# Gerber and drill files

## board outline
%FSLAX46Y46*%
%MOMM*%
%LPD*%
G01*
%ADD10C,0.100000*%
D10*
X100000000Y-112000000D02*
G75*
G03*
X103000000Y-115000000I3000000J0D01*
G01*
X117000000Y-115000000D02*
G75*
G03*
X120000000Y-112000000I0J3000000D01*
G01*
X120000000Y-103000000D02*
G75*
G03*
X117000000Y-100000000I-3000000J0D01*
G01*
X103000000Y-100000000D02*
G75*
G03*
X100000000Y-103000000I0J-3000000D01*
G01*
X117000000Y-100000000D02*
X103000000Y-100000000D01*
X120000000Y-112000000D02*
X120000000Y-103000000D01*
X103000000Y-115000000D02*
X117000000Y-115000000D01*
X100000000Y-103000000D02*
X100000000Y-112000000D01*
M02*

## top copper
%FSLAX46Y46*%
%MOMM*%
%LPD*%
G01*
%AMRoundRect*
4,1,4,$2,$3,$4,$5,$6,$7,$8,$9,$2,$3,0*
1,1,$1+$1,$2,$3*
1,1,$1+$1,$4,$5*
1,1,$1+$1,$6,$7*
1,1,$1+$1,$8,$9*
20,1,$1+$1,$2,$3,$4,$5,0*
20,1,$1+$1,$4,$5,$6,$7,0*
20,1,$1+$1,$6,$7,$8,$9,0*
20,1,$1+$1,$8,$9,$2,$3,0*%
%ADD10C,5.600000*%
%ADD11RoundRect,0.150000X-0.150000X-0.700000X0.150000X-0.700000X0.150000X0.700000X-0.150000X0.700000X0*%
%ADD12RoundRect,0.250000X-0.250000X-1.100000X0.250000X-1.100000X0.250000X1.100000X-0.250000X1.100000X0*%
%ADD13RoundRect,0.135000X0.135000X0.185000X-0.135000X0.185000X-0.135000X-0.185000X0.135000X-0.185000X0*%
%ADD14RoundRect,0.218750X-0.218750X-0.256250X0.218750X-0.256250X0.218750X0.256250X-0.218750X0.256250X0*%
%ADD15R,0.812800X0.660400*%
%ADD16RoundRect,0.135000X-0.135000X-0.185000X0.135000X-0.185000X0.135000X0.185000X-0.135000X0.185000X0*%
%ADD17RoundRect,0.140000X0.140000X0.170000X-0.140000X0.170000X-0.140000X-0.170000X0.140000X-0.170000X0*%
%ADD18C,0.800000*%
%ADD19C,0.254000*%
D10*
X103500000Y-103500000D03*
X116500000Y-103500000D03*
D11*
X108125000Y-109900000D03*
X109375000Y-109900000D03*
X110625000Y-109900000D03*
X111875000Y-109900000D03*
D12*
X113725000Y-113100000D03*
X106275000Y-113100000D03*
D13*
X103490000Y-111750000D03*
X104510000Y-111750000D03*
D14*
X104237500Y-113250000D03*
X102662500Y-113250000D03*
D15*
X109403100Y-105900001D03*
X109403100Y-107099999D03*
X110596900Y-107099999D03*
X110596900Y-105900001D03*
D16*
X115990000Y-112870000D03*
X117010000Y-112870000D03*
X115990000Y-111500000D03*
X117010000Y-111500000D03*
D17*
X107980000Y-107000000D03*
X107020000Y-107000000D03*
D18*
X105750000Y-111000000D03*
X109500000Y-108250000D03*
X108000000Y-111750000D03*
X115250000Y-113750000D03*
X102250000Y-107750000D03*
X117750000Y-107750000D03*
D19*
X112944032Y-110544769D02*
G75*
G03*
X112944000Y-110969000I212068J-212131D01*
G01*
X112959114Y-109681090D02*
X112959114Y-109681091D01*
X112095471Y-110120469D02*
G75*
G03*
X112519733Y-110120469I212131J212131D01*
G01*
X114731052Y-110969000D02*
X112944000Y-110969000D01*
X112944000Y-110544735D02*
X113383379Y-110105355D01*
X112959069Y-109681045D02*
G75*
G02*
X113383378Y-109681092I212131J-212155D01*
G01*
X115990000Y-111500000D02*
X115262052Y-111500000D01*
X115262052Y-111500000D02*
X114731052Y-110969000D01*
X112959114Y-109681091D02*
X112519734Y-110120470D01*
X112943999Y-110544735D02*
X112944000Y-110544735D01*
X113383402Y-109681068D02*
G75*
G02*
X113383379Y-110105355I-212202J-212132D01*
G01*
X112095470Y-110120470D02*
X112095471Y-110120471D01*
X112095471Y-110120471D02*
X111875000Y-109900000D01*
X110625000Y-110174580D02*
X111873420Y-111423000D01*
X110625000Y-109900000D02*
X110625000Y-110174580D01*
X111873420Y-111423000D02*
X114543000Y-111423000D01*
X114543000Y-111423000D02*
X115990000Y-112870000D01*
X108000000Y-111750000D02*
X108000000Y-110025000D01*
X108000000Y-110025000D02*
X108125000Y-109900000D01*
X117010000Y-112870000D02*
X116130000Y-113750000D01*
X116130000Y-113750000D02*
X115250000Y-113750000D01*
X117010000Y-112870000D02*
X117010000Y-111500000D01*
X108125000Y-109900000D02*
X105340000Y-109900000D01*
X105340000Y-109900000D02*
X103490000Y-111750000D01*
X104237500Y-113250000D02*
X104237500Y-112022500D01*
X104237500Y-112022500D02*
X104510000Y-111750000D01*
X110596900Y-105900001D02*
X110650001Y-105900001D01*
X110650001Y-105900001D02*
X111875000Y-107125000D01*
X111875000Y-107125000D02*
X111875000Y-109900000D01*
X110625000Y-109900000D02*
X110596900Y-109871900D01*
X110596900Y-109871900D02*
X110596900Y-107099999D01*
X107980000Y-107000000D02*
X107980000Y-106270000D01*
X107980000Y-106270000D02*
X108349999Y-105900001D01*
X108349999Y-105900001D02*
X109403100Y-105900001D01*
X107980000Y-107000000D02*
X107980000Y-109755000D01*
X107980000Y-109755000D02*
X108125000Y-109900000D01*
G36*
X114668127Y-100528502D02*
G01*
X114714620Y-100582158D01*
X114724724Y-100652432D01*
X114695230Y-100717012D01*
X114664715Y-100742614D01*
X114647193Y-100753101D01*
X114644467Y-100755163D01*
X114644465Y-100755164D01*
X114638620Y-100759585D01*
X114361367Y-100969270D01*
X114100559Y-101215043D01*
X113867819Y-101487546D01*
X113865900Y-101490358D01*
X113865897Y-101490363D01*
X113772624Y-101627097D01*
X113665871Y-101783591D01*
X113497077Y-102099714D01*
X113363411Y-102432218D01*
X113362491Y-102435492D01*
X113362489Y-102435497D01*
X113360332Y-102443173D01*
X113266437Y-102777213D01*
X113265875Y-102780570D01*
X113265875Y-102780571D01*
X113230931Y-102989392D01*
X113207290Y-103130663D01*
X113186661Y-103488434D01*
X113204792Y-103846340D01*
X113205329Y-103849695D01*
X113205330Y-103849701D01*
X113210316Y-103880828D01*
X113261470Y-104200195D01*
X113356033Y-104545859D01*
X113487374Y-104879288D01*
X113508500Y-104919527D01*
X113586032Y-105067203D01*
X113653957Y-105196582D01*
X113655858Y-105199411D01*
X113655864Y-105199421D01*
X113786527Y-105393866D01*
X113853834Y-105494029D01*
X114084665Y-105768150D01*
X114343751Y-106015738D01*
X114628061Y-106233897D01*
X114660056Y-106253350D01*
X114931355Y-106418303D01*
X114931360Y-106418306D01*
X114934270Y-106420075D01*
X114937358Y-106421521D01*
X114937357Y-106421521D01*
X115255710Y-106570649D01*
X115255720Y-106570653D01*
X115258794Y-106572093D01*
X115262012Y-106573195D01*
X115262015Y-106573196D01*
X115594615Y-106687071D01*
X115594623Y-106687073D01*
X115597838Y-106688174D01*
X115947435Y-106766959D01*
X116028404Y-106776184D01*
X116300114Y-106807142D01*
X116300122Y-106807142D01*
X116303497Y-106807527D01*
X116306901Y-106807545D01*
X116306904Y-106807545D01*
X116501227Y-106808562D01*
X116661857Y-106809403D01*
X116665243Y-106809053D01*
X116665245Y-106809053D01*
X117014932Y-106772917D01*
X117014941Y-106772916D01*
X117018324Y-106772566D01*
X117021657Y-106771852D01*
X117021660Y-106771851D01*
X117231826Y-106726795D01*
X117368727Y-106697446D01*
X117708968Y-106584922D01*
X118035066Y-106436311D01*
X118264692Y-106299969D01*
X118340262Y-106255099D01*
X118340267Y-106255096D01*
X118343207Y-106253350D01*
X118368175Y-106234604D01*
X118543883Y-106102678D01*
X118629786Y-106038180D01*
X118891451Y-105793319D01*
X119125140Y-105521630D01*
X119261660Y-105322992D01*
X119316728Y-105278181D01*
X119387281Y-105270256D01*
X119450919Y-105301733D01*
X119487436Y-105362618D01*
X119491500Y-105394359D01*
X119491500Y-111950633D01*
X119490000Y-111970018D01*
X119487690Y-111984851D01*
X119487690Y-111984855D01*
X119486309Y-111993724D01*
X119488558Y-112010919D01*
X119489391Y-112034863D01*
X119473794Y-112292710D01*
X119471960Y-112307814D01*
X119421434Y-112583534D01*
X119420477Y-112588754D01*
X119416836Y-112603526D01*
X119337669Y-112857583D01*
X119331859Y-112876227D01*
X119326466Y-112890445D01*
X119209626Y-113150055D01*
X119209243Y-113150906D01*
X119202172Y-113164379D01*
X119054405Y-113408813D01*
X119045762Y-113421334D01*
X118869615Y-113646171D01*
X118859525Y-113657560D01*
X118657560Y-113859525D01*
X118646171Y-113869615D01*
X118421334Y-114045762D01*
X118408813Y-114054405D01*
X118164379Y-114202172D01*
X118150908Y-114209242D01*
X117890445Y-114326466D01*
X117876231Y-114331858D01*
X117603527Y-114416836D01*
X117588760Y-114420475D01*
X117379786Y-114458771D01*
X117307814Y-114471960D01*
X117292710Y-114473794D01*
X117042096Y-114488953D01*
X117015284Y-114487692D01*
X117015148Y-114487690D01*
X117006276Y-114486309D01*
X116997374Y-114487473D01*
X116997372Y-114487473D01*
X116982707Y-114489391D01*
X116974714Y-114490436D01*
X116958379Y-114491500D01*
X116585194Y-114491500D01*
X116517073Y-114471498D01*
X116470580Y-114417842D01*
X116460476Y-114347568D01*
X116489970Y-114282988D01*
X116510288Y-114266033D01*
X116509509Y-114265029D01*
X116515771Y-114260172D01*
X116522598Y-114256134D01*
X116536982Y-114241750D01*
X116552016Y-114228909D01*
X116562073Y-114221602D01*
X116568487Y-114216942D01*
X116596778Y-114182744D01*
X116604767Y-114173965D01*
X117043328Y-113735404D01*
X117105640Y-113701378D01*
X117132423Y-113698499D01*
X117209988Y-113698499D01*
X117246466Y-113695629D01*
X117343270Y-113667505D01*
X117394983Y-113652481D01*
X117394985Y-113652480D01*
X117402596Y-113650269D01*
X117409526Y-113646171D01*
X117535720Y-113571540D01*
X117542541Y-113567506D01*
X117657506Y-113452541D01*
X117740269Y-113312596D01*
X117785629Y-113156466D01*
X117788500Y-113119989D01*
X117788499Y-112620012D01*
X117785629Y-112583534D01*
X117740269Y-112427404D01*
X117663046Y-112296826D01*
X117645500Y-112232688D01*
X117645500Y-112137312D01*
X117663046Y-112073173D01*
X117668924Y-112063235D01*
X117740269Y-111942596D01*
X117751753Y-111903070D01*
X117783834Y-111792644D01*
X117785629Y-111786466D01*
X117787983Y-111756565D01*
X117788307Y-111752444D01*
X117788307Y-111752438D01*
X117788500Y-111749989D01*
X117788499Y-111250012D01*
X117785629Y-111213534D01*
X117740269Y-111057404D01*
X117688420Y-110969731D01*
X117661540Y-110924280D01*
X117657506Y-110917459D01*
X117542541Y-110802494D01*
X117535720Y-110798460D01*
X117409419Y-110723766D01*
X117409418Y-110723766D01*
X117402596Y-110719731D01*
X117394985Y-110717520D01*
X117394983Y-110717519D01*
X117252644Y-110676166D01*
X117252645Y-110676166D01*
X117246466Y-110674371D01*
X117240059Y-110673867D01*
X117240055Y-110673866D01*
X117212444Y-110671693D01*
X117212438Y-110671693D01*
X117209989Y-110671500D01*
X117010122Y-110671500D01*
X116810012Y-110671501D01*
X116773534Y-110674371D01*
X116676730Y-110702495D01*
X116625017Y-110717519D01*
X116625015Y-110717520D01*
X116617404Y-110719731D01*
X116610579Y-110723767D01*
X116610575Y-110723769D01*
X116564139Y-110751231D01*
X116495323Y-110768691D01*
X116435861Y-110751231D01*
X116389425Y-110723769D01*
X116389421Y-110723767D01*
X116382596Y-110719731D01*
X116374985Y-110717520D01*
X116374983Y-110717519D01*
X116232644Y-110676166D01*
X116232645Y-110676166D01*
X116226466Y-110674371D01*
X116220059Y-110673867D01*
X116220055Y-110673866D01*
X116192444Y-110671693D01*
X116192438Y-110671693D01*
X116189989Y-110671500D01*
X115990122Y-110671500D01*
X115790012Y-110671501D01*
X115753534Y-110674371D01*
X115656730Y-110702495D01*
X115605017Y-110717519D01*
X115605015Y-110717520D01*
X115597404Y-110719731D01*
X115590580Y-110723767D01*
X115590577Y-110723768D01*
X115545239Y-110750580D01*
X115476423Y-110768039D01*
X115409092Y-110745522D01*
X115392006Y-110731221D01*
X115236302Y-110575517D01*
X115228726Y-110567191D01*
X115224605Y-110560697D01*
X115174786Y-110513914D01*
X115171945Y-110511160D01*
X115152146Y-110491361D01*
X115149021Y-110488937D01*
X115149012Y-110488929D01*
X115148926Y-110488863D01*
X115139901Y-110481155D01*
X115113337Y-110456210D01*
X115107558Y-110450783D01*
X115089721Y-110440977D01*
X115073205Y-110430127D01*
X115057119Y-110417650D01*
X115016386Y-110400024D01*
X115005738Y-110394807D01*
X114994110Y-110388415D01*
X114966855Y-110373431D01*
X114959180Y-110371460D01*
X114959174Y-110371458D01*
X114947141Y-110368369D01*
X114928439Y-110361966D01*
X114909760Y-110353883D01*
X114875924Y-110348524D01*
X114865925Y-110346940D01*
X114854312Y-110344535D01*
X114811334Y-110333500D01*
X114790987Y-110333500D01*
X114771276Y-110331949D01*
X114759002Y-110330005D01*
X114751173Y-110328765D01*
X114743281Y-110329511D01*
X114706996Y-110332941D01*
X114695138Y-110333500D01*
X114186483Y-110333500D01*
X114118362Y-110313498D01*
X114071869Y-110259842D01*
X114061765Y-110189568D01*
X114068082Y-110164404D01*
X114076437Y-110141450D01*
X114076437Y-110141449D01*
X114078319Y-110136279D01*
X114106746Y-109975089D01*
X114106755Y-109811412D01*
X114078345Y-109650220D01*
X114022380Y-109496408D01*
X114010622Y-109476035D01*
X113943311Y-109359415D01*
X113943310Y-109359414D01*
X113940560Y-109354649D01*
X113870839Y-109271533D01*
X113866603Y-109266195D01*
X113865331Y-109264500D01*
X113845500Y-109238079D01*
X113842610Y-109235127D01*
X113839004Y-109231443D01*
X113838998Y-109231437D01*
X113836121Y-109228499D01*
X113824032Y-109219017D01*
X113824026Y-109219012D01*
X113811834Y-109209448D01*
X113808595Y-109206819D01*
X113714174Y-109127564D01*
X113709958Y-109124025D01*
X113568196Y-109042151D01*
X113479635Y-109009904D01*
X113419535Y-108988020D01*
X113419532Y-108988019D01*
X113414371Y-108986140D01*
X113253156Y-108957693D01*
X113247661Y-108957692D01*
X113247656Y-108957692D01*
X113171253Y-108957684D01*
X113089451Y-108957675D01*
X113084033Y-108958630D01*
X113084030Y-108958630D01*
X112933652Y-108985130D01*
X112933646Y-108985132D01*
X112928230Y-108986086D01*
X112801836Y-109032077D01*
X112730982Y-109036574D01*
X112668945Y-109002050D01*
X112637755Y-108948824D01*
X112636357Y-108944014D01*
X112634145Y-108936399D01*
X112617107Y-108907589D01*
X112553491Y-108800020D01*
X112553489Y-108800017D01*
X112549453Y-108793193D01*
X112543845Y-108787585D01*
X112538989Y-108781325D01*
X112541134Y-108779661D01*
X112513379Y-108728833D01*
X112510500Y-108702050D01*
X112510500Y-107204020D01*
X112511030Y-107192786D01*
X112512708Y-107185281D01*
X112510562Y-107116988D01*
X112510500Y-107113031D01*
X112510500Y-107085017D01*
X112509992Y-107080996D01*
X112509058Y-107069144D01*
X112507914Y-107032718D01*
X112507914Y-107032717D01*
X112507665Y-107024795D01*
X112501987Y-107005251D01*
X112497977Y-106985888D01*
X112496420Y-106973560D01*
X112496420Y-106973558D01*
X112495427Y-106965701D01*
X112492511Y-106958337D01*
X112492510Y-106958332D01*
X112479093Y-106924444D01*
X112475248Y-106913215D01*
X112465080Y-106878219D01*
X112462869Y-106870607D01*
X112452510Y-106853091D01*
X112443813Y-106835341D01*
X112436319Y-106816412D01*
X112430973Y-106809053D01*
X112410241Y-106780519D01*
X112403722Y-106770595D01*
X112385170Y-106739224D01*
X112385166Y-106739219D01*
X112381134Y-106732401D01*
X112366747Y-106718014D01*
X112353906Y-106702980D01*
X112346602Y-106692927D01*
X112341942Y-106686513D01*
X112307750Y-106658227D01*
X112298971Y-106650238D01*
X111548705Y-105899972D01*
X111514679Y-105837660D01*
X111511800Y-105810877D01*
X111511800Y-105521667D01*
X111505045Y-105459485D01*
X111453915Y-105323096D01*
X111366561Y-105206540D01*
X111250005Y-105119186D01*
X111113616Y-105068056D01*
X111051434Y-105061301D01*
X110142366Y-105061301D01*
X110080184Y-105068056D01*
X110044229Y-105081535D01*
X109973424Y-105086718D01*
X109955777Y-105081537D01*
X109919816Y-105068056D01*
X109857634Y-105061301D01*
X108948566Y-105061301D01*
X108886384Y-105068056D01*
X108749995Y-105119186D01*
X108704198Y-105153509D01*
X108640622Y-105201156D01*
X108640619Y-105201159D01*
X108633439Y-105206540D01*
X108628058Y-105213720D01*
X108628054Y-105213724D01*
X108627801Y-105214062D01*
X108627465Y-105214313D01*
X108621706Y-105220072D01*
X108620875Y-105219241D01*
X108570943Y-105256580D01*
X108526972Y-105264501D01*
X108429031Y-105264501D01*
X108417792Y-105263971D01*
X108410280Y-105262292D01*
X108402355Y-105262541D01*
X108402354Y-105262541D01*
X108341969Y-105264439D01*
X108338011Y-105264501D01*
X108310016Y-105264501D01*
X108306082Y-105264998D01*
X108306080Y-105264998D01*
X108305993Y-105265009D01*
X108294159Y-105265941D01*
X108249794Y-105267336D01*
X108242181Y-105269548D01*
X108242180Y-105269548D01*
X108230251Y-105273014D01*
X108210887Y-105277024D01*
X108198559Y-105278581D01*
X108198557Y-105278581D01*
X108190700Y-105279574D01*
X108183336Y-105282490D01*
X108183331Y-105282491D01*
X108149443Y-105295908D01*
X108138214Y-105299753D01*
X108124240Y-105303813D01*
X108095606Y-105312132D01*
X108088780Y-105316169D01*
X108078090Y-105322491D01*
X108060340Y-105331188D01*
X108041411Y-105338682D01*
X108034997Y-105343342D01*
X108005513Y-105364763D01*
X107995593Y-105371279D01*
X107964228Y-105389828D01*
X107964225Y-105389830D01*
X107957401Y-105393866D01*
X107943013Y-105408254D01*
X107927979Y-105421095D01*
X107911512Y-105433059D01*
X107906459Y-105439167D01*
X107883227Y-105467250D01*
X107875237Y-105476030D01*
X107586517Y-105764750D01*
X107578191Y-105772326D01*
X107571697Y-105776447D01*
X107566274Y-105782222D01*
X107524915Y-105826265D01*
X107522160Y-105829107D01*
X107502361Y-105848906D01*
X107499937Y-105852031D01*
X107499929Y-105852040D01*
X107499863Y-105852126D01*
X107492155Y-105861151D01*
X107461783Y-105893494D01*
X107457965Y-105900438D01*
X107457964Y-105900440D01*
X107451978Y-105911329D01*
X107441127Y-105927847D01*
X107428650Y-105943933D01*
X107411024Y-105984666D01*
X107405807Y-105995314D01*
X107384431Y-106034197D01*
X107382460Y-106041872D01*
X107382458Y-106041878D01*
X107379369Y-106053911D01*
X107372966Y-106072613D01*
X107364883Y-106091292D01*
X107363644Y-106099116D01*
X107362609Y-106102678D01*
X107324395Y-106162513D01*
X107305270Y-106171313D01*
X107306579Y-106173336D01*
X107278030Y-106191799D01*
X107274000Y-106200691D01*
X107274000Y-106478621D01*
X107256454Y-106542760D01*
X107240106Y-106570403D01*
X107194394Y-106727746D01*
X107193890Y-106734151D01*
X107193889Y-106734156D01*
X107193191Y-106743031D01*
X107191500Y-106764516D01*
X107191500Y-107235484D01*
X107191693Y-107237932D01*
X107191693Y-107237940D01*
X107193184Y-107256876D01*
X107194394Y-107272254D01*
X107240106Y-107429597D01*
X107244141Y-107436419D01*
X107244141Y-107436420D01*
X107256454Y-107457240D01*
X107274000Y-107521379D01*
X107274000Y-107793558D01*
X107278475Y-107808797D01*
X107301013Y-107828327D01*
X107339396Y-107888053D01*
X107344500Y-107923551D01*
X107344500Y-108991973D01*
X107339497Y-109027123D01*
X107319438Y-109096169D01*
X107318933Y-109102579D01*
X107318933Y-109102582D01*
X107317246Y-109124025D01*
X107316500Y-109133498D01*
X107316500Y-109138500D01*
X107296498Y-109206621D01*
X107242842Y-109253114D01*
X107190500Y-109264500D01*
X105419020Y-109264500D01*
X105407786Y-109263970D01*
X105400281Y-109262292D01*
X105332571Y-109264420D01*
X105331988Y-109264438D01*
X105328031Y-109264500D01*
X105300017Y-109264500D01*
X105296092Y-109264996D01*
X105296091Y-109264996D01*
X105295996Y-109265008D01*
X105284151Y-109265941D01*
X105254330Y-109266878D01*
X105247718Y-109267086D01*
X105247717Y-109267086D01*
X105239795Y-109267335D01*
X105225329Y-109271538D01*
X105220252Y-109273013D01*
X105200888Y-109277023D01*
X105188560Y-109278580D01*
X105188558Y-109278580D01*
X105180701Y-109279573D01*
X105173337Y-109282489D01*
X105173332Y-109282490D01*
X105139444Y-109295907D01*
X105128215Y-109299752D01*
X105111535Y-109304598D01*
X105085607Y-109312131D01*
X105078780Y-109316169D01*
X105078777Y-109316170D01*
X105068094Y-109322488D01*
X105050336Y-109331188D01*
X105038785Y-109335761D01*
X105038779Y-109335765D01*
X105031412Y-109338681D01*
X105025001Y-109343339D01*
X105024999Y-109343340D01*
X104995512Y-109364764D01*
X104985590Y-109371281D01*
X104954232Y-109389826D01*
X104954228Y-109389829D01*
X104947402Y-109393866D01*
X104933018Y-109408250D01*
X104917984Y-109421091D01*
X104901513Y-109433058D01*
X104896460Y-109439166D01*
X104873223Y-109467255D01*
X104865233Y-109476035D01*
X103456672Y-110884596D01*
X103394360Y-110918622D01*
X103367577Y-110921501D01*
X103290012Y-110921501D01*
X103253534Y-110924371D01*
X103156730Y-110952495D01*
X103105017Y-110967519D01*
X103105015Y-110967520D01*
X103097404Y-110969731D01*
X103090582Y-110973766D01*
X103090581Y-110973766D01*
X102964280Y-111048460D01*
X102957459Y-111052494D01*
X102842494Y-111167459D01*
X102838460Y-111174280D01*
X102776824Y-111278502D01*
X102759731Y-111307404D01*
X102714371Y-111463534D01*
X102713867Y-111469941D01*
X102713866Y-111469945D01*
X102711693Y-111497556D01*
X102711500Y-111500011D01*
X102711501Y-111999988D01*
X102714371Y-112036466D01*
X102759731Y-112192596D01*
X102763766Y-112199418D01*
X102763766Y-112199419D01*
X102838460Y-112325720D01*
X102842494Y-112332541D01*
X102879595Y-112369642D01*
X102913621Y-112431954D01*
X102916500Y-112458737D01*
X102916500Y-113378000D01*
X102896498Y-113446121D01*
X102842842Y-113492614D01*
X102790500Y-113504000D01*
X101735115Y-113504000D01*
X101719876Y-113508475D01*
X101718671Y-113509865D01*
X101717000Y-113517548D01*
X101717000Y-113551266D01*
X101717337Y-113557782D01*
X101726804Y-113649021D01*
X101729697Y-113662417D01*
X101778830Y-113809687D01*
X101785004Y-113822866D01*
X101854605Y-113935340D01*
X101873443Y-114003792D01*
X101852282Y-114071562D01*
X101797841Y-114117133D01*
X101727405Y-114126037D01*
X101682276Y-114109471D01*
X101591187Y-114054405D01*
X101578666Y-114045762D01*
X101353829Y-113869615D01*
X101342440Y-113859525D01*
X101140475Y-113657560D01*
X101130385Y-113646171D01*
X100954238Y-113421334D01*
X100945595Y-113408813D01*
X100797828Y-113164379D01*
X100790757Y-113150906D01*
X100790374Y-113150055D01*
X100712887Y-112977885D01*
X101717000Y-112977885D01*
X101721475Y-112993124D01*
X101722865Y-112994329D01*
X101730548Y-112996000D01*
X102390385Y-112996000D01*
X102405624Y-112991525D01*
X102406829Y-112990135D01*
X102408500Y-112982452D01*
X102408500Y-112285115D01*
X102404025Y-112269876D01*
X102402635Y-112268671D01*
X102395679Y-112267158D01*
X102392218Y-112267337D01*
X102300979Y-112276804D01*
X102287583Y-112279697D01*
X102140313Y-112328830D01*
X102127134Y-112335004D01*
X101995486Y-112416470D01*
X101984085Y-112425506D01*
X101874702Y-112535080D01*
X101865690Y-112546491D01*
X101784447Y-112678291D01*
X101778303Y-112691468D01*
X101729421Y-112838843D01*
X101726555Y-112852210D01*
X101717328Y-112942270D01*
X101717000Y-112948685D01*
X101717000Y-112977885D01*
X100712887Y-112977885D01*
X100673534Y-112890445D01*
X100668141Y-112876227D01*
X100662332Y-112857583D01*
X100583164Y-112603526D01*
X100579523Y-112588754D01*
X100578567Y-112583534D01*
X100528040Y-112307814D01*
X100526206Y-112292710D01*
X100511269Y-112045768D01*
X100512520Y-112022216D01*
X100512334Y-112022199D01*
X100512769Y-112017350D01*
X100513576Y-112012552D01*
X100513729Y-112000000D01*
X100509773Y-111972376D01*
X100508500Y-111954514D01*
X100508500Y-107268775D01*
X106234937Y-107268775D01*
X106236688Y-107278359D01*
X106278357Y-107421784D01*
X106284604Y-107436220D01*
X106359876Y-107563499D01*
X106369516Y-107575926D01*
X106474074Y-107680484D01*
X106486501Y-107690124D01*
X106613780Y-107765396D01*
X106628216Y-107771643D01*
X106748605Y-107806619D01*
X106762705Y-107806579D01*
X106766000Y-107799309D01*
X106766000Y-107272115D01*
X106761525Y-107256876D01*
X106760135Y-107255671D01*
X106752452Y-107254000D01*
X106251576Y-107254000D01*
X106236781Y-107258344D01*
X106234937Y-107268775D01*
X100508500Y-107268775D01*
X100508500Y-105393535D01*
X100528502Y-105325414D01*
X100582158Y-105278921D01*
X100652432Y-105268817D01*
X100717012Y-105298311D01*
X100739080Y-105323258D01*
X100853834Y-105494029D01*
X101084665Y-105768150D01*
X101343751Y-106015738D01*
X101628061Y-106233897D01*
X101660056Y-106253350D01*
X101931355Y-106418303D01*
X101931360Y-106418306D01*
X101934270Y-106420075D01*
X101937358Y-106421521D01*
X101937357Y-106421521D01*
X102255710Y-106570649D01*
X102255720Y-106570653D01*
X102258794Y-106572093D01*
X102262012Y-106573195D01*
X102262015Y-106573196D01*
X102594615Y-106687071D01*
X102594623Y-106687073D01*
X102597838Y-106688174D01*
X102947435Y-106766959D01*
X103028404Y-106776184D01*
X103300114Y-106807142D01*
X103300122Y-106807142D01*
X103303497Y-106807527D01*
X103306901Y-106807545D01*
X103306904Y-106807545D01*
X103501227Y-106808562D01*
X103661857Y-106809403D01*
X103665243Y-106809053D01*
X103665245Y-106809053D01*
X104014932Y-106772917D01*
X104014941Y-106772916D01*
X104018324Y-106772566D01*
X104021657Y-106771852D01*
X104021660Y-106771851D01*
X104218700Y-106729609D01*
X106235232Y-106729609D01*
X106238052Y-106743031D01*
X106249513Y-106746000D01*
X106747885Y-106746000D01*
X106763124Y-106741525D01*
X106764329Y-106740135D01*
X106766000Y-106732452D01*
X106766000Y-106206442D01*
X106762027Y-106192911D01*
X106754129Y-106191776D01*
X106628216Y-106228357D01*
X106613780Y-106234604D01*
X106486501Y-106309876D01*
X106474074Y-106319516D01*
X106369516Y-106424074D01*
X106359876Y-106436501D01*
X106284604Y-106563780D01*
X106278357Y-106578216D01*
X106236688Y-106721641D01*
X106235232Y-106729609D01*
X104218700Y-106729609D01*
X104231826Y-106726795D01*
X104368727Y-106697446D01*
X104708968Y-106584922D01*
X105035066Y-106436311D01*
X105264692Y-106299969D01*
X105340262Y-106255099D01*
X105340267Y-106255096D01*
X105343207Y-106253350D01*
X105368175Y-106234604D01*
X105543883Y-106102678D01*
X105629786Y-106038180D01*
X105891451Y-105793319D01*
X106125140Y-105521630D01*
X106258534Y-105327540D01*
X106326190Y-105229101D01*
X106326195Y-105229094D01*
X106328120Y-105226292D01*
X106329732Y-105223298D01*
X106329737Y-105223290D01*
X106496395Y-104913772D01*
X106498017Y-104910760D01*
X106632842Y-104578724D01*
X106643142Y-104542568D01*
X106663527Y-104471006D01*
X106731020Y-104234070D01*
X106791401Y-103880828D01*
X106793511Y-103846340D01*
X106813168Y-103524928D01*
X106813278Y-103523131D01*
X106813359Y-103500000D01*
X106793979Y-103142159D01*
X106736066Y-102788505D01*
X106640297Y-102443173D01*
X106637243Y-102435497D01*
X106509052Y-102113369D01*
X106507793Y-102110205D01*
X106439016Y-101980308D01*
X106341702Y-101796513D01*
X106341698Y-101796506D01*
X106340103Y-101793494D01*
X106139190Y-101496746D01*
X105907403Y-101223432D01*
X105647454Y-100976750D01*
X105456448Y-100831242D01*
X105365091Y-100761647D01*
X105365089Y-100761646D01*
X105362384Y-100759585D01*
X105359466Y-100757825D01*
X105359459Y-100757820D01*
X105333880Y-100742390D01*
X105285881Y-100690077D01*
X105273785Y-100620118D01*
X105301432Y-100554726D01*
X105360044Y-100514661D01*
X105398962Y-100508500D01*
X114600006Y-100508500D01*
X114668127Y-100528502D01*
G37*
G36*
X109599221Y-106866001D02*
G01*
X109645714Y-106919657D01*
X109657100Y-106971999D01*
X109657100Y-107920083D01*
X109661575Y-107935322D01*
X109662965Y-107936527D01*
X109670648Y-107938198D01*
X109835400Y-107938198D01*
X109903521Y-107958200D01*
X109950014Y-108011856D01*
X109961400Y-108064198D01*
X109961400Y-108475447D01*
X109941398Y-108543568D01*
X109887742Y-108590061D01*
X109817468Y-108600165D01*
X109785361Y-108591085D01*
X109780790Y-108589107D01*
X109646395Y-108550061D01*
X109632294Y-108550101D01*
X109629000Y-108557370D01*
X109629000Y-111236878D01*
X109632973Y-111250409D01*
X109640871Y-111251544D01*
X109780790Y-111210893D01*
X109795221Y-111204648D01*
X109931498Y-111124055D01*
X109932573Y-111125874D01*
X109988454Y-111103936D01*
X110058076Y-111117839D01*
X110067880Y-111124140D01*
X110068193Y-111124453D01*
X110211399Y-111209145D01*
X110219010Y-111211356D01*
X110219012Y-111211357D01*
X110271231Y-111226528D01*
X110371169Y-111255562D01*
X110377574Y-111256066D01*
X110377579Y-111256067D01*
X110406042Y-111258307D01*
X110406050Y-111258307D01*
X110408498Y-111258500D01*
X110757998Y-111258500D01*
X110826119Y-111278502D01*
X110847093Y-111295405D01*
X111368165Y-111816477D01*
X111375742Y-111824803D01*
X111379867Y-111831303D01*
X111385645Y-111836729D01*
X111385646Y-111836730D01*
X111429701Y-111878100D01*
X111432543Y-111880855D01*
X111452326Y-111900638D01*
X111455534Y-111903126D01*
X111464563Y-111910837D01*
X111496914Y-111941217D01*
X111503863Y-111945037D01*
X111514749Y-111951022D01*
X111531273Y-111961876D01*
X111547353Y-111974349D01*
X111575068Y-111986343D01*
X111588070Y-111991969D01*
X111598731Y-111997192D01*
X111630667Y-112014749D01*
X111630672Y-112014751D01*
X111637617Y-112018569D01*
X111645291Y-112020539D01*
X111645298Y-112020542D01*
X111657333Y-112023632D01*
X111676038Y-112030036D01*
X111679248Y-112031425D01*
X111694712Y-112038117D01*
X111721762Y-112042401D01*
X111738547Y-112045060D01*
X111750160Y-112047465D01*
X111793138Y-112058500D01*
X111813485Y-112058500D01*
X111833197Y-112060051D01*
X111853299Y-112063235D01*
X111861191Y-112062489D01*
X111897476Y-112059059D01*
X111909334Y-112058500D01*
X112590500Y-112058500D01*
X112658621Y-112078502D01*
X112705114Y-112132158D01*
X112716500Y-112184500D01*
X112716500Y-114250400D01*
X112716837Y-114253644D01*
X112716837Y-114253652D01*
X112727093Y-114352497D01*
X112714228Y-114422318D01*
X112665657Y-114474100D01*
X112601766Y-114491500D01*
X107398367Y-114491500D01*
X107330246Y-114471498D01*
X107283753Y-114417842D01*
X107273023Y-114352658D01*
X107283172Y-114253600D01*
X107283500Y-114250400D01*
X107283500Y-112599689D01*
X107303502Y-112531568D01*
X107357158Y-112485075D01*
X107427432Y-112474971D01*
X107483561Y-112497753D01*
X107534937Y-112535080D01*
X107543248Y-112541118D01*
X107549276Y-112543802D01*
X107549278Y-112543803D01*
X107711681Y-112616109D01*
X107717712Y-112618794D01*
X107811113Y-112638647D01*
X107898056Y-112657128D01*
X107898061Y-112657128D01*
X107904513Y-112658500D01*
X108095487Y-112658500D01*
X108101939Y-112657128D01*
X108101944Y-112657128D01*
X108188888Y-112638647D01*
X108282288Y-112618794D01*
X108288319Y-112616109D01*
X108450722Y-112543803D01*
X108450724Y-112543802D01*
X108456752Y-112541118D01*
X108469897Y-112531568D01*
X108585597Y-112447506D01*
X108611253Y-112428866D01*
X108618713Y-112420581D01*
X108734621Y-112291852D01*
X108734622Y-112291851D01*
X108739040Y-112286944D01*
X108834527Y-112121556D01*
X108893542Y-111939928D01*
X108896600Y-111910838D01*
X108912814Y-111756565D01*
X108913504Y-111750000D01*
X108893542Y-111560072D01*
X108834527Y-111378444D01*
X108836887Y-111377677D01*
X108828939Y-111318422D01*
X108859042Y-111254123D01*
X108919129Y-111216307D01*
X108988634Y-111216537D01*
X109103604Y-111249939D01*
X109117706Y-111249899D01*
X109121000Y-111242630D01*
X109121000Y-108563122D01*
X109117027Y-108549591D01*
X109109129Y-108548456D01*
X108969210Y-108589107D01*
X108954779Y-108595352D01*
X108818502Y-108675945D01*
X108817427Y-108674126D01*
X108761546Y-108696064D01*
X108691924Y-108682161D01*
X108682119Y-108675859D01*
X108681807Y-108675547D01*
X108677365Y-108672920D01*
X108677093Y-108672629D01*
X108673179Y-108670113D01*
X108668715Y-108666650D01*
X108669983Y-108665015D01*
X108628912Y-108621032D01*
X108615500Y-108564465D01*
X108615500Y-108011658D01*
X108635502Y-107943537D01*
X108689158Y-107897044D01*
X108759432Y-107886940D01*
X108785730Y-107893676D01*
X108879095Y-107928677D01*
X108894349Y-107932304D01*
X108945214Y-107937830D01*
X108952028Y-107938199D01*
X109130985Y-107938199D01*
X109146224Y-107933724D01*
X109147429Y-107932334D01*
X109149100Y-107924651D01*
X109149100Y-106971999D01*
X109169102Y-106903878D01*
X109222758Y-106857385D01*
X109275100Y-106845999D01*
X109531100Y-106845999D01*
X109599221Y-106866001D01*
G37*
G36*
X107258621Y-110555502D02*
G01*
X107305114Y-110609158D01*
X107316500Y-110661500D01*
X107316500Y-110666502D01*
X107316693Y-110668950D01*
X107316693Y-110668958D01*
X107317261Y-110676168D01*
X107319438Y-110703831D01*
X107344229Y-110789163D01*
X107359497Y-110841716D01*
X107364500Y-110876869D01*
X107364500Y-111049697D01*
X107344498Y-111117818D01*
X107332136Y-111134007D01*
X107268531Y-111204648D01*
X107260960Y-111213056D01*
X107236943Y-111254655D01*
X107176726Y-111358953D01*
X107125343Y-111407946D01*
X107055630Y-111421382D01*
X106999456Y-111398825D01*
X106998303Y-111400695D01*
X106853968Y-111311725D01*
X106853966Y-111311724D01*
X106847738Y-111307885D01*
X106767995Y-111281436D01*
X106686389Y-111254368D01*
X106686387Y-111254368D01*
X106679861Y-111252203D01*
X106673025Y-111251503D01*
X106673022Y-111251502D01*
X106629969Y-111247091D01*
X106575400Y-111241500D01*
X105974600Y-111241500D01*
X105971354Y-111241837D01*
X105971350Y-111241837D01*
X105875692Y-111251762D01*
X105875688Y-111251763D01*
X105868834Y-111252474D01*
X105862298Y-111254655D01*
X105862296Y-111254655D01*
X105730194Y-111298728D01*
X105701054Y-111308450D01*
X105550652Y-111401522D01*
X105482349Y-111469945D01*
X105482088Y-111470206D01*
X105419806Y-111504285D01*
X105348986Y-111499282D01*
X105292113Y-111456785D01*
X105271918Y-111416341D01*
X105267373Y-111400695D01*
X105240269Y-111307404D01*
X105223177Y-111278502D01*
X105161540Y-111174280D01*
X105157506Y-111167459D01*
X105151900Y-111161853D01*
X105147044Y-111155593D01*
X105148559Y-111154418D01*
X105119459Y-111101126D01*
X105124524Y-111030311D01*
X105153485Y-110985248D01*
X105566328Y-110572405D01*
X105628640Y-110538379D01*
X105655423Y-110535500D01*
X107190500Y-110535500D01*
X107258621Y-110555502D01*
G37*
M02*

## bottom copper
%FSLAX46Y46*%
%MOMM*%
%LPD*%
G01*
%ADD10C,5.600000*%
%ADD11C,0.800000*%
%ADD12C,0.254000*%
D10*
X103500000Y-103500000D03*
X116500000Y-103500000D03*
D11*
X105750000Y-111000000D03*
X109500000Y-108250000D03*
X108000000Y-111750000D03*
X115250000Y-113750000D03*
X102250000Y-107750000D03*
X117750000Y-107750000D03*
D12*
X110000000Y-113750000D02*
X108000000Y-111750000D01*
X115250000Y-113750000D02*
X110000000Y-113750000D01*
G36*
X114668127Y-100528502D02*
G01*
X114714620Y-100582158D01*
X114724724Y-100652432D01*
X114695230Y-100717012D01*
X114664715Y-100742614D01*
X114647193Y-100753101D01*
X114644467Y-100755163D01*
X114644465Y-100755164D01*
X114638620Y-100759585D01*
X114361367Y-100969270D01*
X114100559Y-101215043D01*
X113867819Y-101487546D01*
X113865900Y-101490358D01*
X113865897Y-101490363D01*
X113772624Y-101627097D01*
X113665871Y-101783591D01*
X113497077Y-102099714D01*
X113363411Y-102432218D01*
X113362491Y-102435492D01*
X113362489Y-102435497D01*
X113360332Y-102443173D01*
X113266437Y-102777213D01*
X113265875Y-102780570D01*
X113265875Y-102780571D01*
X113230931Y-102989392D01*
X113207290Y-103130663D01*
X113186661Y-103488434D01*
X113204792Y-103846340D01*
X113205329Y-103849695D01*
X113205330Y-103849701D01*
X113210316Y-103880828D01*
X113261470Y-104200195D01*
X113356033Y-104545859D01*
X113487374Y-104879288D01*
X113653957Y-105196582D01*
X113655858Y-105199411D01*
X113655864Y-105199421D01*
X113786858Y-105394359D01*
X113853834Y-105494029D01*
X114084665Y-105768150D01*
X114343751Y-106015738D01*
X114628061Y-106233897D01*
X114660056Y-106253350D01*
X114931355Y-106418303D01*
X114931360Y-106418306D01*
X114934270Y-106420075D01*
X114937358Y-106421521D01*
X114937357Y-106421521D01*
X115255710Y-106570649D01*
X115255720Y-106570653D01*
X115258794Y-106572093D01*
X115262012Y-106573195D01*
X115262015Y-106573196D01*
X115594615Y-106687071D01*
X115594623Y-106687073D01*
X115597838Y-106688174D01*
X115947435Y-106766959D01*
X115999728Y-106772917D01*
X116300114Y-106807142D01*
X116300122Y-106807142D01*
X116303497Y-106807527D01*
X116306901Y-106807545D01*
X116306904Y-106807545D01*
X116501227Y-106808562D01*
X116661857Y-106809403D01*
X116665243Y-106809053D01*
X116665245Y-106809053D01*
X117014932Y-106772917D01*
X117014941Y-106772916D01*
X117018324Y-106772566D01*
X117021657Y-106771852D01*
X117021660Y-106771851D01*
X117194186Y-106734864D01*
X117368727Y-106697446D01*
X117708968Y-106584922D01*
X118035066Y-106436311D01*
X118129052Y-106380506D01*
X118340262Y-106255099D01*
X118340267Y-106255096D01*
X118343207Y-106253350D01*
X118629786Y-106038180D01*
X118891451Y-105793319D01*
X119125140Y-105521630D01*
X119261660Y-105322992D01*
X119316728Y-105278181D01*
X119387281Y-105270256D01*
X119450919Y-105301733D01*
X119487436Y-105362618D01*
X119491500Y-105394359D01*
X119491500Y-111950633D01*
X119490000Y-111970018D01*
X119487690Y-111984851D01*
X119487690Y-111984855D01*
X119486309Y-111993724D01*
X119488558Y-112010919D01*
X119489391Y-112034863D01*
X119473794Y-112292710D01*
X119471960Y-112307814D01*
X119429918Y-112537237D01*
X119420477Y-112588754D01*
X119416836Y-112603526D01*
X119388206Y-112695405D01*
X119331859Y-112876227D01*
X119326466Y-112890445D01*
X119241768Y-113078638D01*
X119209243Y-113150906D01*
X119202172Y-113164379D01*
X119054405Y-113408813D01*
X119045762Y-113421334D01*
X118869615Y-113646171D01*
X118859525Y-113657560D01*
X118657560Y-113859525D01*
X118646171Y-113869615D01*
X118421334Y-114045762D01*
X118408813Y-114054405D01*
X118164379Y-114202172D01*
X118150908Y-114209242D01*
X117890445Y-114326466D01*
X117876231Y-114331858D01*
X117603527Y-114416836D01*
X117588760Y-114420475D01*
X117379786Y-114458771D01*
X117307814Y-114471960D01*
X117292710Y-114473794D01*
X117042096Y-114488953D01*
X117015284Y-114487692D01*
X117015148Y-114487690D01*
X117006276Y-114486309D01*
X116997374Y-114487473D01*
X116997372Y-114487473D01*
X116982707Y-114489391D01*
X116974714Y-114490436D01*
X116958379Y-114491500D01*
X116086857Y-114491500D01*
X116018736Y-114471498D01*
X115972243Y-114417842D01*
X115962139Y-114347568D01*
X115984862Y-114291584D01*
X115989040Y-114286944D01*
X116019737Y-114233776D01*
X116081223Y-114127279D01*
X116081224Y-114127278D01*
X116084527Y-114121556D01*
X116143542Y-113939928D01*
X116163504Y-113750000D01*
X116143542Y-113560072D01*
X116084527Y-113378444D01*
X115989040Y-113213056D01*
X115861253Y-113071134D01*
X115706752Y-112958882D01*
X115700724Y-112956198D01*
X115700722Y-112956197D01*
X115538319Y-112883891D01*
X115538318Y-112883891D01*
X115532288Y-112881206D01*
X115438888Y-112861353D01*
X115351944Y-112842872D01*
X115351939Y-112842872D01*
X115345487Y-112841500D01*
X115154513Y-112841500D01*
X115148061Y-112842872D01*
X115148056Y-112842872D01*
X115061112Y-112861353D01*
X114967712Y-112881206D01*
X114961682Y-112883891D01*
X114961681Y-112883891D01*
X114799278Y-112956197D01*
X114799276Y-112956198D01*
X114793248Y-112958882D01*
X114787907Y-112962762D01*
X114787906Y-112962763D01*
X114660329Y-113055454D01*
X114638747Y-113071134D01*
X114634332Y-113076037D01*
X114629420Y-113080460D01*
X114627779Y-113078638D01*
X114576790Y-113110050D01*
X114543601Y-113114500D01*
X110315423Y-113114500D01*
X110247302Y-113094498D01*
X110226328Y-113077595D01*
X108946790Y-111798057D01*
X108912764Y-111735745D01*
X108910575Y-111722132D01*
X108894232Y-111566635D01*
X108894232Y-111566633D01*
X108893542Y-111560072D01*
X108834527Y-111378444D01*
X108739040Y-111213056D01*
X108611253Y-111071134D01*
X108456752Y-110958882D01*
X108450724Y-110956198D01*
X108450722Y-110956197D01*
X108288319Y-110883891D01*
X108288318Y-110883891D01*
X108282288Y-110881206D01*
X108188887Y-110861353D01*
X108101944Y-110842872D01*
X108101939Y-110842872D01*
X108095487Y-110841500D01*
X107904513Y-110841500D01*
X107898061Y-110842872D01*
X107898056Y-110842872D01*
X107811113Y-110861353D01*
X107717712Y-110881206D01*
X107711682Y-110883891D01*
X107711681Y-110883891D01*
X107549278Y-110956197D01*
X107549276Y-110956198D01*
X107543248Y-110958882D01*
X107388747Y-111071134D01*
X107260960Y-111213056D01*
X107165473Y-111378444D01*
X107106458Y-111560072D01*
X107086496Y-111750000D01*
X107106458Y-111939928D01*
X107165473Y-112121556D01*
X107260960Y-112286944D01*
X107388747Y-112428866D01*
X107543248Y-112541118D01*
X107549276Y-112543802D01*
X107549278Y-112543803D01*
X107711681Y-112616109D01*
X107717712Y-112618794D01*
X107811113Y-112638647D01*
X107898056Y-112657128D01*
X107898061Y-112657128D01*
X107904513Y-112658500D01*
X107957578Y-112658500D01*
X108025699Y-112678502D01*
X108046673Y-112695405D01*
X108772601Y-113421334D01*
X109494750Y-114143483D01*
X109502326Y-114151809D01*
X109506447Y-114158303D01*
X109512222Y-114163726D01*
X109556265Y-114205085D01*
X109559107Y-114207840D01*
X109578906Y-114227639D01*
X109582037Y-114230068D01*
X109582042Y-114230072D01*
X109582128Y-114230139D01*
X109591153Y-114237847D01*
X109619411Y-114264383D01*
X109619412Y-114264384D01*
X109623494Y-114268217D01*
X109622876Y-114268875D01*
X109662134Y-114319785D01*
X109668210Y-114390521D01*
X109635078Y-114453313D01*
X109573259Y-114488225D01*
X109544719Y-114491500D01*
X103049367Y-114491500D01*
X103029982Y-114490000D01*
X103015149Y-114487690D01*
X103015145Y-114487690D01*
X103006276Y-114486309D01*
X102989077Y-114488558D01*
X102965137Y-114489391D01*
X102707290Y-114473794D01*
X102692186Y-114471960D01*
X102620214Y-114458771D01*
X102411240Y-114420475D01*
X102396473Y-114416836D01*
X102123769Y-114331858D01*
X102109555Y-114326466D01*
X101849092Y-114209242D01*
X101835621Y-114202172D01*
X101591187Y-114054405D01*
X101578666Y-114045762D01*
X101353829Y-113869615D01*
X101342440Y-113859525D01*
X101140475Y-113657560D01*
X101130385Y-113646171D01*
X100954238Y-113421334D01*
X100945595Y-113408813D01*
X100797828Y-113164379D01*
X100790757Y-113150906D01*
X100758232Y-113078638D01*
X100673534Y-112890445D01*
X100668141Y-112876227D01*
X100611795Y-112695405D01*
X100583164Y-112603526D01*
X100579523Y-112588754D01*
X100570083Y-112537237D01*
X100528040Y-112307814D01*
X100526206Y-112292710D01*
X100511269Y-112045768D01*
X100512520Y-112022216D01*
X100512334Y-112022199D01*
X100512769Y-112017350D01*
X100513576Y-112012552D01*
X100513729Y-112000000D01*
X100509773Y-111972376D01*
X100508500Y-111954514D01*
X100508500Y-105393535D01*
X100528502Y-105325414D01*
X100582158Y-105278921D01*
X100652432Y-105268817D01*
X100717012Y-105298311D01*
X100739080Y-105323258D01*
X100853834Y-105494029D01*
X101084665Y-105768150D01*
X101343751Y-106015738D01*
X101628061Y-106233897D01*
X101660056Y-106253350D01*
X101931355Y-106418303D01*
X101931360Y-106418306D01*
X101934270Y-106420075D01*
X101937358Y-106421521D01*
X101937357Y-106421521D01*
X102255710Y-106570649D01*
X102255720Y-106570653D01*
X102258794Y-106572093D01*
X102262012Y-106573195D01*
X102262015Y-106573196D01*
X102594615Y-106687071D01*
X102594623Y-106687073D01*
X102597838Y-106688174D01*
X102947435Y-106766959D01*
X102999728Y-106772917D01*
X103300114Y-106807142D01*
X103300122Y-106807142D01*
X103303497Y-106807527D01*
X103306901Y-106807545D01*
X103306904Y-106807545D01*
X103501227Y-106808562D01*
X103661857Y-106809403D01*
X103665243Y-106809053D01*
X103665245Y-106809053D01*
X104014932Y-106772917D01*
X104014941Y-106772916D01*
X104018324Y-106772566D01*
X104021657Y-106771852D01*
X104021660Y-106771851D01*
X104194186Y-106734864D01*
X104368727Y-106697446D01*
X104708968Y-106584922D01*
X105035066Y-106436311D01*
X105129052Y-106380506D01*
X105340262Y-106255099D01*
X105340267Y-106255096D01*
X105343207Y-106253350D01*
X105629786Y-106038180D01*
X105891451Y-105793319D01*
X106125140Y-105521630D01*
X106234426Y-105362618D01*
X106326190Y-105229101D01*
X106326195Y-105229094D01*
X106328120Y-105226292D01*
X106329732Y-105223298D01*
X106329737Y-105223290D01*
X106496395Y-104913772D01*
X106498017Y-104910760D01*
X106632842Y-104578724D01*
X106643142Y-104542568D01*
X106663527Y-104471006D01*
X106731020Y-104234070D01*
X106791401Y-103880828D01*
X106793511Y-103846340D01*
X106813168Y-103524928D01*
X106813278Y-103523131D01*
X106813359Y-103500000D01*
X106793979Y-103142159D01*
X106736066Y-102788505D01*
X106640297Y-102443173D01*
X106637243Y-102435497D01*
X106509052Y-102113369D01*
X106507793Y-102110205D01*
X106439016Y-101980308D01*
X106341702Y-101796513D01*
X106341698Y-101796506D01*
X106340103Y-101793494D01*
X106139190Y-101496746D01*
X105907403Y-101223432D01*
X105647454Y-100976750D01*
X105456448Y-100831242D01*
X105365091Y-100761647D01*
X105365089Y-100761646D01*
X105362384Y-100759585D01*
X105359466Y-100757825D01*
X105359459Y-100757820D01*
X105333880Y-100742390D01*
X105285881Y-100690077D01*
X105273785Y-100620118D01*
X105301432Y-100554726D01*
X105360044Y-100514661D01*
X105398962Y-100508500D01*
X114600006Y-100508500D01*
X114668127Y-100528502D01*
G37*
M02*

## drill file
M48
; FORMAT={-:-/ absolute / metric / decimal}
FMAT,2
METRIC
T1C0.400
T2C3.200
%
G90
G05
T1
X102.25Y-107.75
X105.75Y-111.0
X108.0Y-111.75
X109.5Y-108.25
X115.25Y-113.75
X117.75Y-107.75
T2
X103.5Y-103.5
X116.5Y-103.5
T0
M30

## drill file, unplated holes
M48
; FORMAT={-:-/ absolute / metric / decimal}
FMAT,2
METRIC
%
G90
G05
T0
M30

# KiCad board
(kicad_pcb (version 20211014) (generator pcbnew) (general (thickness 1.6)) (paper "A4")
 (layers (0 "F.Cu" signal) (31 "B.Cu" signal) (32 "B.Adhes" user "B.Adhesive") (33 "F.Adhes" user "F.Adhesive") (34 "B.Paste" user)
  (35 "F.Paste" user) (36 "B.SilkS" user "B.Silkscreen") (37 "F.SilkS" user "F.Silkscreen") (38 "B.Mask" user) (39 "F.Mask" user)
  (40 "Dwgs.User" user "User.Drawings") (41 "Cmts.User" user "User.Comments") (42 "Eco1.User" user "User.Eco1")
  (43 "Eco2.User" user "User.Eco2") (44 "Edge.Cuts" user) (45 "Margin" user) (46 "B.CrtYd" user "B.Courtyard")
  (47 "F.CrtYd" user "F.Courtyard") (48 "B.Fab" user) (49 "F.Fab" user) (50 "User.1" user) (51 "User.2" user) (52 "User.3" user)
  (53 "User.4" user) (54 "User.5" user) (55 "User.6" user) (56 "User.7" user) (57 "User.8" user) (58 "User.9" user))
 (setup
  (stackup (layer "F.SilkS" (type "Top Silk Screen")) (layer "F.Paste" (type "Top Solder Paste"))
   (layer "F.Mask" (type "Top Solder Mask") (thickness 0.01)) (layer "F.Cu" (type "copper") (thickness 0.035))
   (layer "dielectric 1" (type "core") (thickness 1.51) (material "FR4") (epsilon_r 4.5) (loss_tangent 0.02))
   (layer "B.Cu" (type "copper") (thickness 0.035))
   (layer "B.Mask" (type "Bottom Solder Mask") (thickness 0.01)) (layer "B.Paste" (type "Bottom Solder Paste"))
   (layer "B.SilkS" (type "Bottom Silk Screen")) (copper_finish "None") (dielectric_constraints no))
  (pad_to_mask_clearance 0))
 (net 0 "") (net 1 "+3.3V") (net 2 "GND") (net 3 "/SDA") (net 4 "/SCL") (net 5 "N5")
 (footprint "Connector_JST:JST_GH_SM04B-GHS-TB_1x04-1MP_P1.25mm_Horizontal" (layer "F.Cu") (at 110 111.75)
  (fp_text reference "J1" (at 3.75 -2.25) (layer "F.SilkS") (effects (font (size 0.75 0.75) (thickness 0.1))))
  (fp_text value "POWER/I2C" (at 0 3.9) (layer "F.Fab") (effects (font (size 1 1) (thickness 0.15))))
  (pad "1" smd roundrect (at -1.875 -1.85) (size 0.6 1.7) (layers "F.Cu" "F.Paste" "F.Mask") (roundrect_rratio 0.25) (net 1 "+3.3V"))
  (pad "2" smd roundrect (at -0.625 -1.85) (size 0.6 1.7) (layers "F.Cu" "F.Paste" "F.Mask") (roundrect_rratio 0.25) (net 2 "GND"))
  (pad "3" smd roundrect (at 0.625 -1.85) (size 0.6 1.7) (layers "F.Cu" "F.Paste" "F.Mask") (roundrect_rratio 0.25) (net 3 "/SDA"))
  (pad "4" smd roundrect (at 1.875 -1.85) (size 0.6 1.7) (layers "F.Cu" "F.Paste" "F.Mask") (roundrect_rratio 0.25) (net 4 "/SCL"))
  (pad "MP" smd roundrect (at 3.725 1.35) (size 1 2.7) (layers "F.Cu" "F.Paste" "F.Mask") (roundrect_rratio 0.25))
  (pad "MP" smd roundrect (at -3.725 1.35) (size 1 2.7) (layers "F.Cu" "F.Paste" "F.Mask") (roundrect_rratio 0.25)))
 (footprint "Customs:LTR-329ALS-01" (layer "F.Cu") (at 110 106.5)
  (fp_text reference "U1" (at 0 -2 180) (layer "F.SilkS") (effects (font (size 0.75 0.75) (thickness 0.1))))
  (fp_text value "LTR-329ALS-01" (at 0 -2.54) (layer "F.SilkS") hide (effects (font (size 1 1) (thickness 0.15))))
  (pad "1" smd rect locked (at -0.5969 -0.599999) (size 0.8128 0.6604) (layers "F.Cu" "F.Paste" "F.Mask") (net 1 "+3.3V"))
  (pad "2" smd rect locked (at -0.5969 0.599999) (size 0.8128 0.6604) (layers "F.Cu" "F.Paste" "F.Mask") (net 2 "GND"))
  (pad "3" smd rect locked (at 0.5969 0.599999) (size 0.8128 0.6604) (layers "F.Cu" "F.Paste" "F.Mask") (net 3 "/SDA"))
  (pad "4" smd rect locked (at 0.5969 -0.599999) (size 0.8128 0.6604) (layers "F.Cu" "F.Paste" "F.Mask") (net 4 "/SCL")))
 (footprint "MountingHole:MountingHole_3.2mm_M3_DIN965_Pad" (layer "F.Cu") (at 116.5 103.5)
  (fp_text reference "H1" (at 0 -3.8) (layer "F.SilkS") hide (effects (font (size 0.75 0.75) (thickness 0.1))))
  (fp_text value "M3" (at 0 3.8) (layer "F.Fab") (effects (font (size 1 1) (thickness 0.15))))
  (pad "1" thru_hole circle (at 0 0) (size 5.6 5.6) (drill 3.2) (layers *.Cu *.Mask)))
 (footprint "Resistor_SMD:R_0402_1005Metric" (layer "F.Cu") (at 116.5 112.87)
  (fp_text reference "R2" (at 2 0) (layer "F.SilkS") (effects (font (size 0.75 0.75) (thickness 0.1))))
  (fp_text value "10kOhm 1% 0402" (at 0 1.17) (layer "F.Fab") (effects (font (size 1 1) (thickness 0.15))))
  (pad "1" smd roundrect (at -0.51 0) (size 0.54 0.64) (layers "F.Cu" "F.Paste" "F.Mask") (roundrect_rratio 0.25) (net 3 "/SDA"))
  (pad "2" smd roundrect (at 0.51 0) (size 0.54 0.64) (layers "F.Cu" "F.Paste" "F.Mask") (roundrect_rratio 0.25) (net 1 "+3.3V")))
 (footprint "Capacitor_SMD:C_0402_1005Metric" (layer "F.Cu") (at 107.5 107 180)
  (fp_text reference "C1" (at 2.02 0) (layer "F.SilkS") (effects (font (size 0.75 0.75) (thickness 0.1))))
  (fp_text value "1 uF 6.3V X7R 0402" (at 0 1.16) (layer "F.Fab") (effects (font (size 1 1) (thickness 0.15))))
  (pad "1" smd roundrect (at -0.48 0 180) (size 0.56 0.62) (layers "F.Cu" "F.Paste" "F.Mask") (roundrect_rratio 0.25) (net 1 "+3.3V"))
  (pad "2" smd roundrect (at 0.48 0 180) (size 0.56 0.62) (layers "F.Cu" "F.Paste" "F.Mask") (roundrect_rratio 0.25) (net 2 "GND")))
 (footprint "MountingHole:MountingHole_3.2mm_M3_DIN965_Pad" (layer "F.Cu") (at 103.5 103.5)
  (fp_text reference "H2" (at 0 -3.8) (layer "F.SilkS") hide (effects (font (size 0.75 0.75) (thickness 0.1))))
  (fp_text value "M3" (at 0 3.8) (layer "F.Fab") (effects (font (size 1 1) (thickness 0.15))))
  (pad "1" thru_hole circle (at 0 0) (size 5.6 5.6) (drill 3.2) (layers *.Cu *.Mask)))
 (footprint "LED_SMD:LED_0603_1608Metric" (layer "F.Cu") (at 103.45 113.25)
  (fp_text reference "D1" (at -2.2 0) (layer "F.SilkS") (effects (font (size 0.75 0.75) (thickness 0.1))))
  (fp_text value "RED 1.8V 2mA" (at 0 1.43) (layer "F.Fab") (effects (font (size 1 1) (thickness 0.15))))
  (pad "1" smd roundrect (at -0.7875 0) (size 0.875 0.95) (layers "F.Cu" "F.Paste" "F.Mask") (roundrect_rratio 0.25) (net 2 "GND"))
  (pad "2" smd roundrect (at 0.7875 0) (size 0.875 0.95) (layers "F.Cu" "F.Paste" "F.Mask") (roundrect_rratio 0.25) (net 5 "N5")))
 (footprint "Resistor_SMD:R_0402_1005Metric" (layer "F.Cu") (at 116.5 111.5)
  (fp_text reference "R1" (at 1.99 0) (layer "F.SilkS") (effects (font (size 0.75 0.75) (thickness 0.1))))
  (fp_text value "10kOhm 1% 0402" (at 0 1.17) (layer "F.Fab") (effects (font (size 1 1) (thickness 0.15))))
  (pad "1" smd roundrect (at -0.51 0) (size 0.54 0.64) (layers "F.Cu" "F.Paste" "F.Mask") (roundrect_rratio 0.25) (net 4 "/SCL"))
  (pad "2" smd roundrect (at 0.51 0) (size 0.54 0.64) (layers "F.Cu" "F.Paste" "F.Mask") (roundrect_rratio 0.25) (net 1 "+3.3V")))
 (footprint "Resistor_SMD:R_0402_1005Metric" (layer "F.Cu") (at 104 111.75 180)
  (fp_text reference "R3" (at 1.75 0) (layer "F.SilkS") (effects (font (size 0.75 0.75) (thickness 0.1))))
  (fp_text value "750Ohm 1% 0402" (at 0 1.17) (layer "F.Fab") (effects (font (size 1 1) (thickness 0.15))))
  (pad "1" smd roundrect (at -0.51 0 180) (size 0.54 0.64) (layers "F.Cu" "F.Paste" "F.Mask") (roundrect_rratio 0.25) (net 5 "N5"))
  (pad "2" smd roundrect (at 0.51 0 180) (size 0.54 0.64) (layers "F.Cu" "F.Paste" "F.Mask") (roundrect_rratio 0.25) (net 1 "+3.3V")))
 (gr_line (start 103 115) (end 117 115) (layer "Edge.Cuts") (width 0.1))
 (gr_arc (start 100 103) (mid 100.87868 100.87868) (end 103 100) (layer "Edge.Cuts") (width 0.1))
 (gr_line (start 100 103) (end 100 112) (layer "Edge.Cuts") (width 0.1))
 (gr_line (start 120 112) (end 120 103) (layer "Edge.Cuts") (width 0.1))
 (gr_line (start 117 100) (end 103 100) (layer "Edge.Cuts") (width 0.1))
 (gr_arc (start 117 100) (mid 119.12132 100.87868) (end 120 103) (layer "Edge.Cuts") (width 0.1))
 (gr_arc (start 103 115) (mid 100.87868 114.12132) (end 100 112) (layer "Edge.Cuts") (width 0.1))
 (gr_arc (start 120 112) (mid 119.12132 114.12132) (end 117 115) (layer "Edge.Cuts") (width 0.1))
 (segment (start 117.01 112.87) (end 116.13 113.75) (width 0.254) (layer "F.Cu") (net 1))
 (segment (start 117.01 112.87) (end 117.01 111.5) (width 0.254) (layer "F.Cu") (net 1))
 (segment (start 116.13 113.75) (end 115.25 113.75) (width 0.254) (layer "F.Cu") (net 1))
 (segment (start 107.98 109.755) (end 108.125 109.9) (width 0.254) (layer "F.Cu") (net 1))
 (segment (start 107.98 106.27) (end 108.349999 105.900001) (width 0.254) (layer "F.Cu") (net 1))
 (segment (start 108.349999 105.900001) (end 109.4031 105.900001) (width 0.254) (layer "F.Cu") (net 1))
 (segment (start 107.98 107) (end 107.98 106.27) (width 0.254) (layer "F.Cu") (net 1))
 (segment (start 105.34 109.9) (end 103.49 111.75) (width 0.254) (layer "F.Cu") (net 1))
 (segment (start 107.98 107) (end 107.98 109.755) (width 0.254) (layer "F.Cu") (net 1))
 (segment (start 108 111.75) (end 108 110.025) (width 0.254) (layer "F.Cu") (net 1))
 (segment (start 108 110.025) (end 108.125 109.9) (width 0.254) (layer "F.Cu") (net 1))
 (segment (start 108.125 109.9) (end 105.34 109.9) (width 0.254) (layer "F.Cu") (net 1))
 (via (at 115.25 113.75) (size 0.8) (drill 0.4) (layers "F.Cu" "B.Cu") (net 1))
 (via (at 108 111.75) (size 0.8) (drill 0.4) (layers "F.Cu" "B.Cu") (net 1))
 (segment (start 115.25 113.75) (end 110 113.75) (width 0.254) (layer "B.Cu") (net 1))
 (segment (start 110 113.75) (end 108 111.75) (width 0.254) (layer "B.Cu") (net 1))
 (via (at 102.25 107.75) (size 0.8) (drill 0.4) (layers "F.Cu" "B.Cu") (free) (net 2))
 (via (at 105.75 111) (size 0.8) (drill 0.4) (layers "F.Cu" "B.Cu") (free) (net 2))
 (via (at 117.75 107.75) (size 0.8) (drill 0.4) (layers "F.Cu" "B.Cu") (free) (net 2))
 (via (at 109.5 108.25) (size 0.8) (drill 0.4) (layers "F.Cu" "B.Cu") (free) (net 2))
 (segment (start 110.5969 109.8719) (end 110.5969 107.099999) (width 0.254) (layer "F.Cu") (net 3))
 (segment (start 110.625 110.17458) (end 111.87342 111.423) (width 0.254) (layer "F.Cu") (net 3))
 (segment (start 111.87342 111.423) (end 114.543 111.423) (width 0.254) (layer "F.Cu") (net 3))
 (segment (start 110.625 109.9) (end 110.625 110.17458) (width 0.254) (layer "F.Cu") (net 3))
 (segment (start 110.625 109.9) (end 110.5969 109.8719) (width 0.254) (layer "F.Cu") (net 3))
 (segment (start 114.543 111.423) (end 115.99 112.87) (width 0.254) (layer "F.Cu") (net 3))
 (segment (start 112.09547 110.12047) (end 112.095471 110.120471) (width 0.254) (layer "F.Cu") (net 4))
 (segment (start 115.99 111.5) (end 115.262052 111.5) (width 0.254) (layer "F.Cu") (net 4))
 (segment (start 111.875 107.125) (end 111.875 109.9) (width 0.254) (layer "F.Cu") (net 4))
 (segment (start 115.262052 111.5) (end 114.731052 110.969) (width 0.254) (layer "F.Cu") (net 4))
 (segment (start 112.959114 109.681091) (end 112.519734 110.12047) (width 0.254) (layer "F.Cu") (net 4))
 (segment (start 110.5969 105.900001) (end 110.650001 105.900001) (width 0.254) (layer "F.Cu") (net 4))
 (segment (start 112.959114 109.68109) (end 112.959114 109.681091) (width 0.254) (layer "F.Cu") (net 4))
 (segment (start 112.943999 110.544735) (end 112.944 110.544735) (width 0.254) (layer "F.Cu") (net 4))
 (segment (start 112.944 110.544735) (end 113.383379 110.105355) (width 0.254) (layer "F.Cu") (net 4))
 (segment (start 114.731052 110.969) (end 112.944 110.969) (width 0.254) (layer "F.Cu") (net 4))
 (segment (start 112.095471 110.120471) (end 111.875 109.9) (width 0.254) (layer "F.Cu") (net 4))
 (segment (start 110.650001 105.900001) (end 111.875 107.125) (width 0.254) (layer "F.Cu") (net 4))
 (arc (start 112.944 110.969) (mid 112.856131 110.756868) (end 112.943999 110.544735) (width 0.254) (layer "F.Cu") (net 4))
 (arc (start 113.383379 110.105355) (mid 113.471247 109.893223) (end 113.383379 109.681091) (width 0.254) (layer "F.Cu") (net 4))
 (arc (start 113.383379 109.681091) (mid 113.171247 109.593222) (end 112.959114 109.68109) (width 0.254) (layer "F.Cu") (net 4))
 (arc (start 112.519734 110.12047) (mid 112.307602 110.208338) (end 112.09547 110.12047) (width 0.254) (layer "F.Cu") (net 4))
 (segment (start 104.2375 112.0225) (end 104.51 111.75) (width 0.254) (layer "F.Cu") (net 5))
 (segment (start 104.2375 113.25) (end 104.2375 112.0225) (width 0.254) (layer "F.Cu") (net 5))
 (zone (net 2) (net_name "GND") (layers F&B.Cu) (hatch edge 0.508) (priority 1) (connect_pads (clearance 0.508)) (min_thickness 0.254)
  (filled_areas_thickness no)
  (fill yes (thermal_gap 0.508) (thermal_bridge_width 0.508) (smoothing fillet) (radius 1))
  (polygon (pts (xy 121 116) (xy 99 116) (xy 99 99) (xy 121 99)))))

